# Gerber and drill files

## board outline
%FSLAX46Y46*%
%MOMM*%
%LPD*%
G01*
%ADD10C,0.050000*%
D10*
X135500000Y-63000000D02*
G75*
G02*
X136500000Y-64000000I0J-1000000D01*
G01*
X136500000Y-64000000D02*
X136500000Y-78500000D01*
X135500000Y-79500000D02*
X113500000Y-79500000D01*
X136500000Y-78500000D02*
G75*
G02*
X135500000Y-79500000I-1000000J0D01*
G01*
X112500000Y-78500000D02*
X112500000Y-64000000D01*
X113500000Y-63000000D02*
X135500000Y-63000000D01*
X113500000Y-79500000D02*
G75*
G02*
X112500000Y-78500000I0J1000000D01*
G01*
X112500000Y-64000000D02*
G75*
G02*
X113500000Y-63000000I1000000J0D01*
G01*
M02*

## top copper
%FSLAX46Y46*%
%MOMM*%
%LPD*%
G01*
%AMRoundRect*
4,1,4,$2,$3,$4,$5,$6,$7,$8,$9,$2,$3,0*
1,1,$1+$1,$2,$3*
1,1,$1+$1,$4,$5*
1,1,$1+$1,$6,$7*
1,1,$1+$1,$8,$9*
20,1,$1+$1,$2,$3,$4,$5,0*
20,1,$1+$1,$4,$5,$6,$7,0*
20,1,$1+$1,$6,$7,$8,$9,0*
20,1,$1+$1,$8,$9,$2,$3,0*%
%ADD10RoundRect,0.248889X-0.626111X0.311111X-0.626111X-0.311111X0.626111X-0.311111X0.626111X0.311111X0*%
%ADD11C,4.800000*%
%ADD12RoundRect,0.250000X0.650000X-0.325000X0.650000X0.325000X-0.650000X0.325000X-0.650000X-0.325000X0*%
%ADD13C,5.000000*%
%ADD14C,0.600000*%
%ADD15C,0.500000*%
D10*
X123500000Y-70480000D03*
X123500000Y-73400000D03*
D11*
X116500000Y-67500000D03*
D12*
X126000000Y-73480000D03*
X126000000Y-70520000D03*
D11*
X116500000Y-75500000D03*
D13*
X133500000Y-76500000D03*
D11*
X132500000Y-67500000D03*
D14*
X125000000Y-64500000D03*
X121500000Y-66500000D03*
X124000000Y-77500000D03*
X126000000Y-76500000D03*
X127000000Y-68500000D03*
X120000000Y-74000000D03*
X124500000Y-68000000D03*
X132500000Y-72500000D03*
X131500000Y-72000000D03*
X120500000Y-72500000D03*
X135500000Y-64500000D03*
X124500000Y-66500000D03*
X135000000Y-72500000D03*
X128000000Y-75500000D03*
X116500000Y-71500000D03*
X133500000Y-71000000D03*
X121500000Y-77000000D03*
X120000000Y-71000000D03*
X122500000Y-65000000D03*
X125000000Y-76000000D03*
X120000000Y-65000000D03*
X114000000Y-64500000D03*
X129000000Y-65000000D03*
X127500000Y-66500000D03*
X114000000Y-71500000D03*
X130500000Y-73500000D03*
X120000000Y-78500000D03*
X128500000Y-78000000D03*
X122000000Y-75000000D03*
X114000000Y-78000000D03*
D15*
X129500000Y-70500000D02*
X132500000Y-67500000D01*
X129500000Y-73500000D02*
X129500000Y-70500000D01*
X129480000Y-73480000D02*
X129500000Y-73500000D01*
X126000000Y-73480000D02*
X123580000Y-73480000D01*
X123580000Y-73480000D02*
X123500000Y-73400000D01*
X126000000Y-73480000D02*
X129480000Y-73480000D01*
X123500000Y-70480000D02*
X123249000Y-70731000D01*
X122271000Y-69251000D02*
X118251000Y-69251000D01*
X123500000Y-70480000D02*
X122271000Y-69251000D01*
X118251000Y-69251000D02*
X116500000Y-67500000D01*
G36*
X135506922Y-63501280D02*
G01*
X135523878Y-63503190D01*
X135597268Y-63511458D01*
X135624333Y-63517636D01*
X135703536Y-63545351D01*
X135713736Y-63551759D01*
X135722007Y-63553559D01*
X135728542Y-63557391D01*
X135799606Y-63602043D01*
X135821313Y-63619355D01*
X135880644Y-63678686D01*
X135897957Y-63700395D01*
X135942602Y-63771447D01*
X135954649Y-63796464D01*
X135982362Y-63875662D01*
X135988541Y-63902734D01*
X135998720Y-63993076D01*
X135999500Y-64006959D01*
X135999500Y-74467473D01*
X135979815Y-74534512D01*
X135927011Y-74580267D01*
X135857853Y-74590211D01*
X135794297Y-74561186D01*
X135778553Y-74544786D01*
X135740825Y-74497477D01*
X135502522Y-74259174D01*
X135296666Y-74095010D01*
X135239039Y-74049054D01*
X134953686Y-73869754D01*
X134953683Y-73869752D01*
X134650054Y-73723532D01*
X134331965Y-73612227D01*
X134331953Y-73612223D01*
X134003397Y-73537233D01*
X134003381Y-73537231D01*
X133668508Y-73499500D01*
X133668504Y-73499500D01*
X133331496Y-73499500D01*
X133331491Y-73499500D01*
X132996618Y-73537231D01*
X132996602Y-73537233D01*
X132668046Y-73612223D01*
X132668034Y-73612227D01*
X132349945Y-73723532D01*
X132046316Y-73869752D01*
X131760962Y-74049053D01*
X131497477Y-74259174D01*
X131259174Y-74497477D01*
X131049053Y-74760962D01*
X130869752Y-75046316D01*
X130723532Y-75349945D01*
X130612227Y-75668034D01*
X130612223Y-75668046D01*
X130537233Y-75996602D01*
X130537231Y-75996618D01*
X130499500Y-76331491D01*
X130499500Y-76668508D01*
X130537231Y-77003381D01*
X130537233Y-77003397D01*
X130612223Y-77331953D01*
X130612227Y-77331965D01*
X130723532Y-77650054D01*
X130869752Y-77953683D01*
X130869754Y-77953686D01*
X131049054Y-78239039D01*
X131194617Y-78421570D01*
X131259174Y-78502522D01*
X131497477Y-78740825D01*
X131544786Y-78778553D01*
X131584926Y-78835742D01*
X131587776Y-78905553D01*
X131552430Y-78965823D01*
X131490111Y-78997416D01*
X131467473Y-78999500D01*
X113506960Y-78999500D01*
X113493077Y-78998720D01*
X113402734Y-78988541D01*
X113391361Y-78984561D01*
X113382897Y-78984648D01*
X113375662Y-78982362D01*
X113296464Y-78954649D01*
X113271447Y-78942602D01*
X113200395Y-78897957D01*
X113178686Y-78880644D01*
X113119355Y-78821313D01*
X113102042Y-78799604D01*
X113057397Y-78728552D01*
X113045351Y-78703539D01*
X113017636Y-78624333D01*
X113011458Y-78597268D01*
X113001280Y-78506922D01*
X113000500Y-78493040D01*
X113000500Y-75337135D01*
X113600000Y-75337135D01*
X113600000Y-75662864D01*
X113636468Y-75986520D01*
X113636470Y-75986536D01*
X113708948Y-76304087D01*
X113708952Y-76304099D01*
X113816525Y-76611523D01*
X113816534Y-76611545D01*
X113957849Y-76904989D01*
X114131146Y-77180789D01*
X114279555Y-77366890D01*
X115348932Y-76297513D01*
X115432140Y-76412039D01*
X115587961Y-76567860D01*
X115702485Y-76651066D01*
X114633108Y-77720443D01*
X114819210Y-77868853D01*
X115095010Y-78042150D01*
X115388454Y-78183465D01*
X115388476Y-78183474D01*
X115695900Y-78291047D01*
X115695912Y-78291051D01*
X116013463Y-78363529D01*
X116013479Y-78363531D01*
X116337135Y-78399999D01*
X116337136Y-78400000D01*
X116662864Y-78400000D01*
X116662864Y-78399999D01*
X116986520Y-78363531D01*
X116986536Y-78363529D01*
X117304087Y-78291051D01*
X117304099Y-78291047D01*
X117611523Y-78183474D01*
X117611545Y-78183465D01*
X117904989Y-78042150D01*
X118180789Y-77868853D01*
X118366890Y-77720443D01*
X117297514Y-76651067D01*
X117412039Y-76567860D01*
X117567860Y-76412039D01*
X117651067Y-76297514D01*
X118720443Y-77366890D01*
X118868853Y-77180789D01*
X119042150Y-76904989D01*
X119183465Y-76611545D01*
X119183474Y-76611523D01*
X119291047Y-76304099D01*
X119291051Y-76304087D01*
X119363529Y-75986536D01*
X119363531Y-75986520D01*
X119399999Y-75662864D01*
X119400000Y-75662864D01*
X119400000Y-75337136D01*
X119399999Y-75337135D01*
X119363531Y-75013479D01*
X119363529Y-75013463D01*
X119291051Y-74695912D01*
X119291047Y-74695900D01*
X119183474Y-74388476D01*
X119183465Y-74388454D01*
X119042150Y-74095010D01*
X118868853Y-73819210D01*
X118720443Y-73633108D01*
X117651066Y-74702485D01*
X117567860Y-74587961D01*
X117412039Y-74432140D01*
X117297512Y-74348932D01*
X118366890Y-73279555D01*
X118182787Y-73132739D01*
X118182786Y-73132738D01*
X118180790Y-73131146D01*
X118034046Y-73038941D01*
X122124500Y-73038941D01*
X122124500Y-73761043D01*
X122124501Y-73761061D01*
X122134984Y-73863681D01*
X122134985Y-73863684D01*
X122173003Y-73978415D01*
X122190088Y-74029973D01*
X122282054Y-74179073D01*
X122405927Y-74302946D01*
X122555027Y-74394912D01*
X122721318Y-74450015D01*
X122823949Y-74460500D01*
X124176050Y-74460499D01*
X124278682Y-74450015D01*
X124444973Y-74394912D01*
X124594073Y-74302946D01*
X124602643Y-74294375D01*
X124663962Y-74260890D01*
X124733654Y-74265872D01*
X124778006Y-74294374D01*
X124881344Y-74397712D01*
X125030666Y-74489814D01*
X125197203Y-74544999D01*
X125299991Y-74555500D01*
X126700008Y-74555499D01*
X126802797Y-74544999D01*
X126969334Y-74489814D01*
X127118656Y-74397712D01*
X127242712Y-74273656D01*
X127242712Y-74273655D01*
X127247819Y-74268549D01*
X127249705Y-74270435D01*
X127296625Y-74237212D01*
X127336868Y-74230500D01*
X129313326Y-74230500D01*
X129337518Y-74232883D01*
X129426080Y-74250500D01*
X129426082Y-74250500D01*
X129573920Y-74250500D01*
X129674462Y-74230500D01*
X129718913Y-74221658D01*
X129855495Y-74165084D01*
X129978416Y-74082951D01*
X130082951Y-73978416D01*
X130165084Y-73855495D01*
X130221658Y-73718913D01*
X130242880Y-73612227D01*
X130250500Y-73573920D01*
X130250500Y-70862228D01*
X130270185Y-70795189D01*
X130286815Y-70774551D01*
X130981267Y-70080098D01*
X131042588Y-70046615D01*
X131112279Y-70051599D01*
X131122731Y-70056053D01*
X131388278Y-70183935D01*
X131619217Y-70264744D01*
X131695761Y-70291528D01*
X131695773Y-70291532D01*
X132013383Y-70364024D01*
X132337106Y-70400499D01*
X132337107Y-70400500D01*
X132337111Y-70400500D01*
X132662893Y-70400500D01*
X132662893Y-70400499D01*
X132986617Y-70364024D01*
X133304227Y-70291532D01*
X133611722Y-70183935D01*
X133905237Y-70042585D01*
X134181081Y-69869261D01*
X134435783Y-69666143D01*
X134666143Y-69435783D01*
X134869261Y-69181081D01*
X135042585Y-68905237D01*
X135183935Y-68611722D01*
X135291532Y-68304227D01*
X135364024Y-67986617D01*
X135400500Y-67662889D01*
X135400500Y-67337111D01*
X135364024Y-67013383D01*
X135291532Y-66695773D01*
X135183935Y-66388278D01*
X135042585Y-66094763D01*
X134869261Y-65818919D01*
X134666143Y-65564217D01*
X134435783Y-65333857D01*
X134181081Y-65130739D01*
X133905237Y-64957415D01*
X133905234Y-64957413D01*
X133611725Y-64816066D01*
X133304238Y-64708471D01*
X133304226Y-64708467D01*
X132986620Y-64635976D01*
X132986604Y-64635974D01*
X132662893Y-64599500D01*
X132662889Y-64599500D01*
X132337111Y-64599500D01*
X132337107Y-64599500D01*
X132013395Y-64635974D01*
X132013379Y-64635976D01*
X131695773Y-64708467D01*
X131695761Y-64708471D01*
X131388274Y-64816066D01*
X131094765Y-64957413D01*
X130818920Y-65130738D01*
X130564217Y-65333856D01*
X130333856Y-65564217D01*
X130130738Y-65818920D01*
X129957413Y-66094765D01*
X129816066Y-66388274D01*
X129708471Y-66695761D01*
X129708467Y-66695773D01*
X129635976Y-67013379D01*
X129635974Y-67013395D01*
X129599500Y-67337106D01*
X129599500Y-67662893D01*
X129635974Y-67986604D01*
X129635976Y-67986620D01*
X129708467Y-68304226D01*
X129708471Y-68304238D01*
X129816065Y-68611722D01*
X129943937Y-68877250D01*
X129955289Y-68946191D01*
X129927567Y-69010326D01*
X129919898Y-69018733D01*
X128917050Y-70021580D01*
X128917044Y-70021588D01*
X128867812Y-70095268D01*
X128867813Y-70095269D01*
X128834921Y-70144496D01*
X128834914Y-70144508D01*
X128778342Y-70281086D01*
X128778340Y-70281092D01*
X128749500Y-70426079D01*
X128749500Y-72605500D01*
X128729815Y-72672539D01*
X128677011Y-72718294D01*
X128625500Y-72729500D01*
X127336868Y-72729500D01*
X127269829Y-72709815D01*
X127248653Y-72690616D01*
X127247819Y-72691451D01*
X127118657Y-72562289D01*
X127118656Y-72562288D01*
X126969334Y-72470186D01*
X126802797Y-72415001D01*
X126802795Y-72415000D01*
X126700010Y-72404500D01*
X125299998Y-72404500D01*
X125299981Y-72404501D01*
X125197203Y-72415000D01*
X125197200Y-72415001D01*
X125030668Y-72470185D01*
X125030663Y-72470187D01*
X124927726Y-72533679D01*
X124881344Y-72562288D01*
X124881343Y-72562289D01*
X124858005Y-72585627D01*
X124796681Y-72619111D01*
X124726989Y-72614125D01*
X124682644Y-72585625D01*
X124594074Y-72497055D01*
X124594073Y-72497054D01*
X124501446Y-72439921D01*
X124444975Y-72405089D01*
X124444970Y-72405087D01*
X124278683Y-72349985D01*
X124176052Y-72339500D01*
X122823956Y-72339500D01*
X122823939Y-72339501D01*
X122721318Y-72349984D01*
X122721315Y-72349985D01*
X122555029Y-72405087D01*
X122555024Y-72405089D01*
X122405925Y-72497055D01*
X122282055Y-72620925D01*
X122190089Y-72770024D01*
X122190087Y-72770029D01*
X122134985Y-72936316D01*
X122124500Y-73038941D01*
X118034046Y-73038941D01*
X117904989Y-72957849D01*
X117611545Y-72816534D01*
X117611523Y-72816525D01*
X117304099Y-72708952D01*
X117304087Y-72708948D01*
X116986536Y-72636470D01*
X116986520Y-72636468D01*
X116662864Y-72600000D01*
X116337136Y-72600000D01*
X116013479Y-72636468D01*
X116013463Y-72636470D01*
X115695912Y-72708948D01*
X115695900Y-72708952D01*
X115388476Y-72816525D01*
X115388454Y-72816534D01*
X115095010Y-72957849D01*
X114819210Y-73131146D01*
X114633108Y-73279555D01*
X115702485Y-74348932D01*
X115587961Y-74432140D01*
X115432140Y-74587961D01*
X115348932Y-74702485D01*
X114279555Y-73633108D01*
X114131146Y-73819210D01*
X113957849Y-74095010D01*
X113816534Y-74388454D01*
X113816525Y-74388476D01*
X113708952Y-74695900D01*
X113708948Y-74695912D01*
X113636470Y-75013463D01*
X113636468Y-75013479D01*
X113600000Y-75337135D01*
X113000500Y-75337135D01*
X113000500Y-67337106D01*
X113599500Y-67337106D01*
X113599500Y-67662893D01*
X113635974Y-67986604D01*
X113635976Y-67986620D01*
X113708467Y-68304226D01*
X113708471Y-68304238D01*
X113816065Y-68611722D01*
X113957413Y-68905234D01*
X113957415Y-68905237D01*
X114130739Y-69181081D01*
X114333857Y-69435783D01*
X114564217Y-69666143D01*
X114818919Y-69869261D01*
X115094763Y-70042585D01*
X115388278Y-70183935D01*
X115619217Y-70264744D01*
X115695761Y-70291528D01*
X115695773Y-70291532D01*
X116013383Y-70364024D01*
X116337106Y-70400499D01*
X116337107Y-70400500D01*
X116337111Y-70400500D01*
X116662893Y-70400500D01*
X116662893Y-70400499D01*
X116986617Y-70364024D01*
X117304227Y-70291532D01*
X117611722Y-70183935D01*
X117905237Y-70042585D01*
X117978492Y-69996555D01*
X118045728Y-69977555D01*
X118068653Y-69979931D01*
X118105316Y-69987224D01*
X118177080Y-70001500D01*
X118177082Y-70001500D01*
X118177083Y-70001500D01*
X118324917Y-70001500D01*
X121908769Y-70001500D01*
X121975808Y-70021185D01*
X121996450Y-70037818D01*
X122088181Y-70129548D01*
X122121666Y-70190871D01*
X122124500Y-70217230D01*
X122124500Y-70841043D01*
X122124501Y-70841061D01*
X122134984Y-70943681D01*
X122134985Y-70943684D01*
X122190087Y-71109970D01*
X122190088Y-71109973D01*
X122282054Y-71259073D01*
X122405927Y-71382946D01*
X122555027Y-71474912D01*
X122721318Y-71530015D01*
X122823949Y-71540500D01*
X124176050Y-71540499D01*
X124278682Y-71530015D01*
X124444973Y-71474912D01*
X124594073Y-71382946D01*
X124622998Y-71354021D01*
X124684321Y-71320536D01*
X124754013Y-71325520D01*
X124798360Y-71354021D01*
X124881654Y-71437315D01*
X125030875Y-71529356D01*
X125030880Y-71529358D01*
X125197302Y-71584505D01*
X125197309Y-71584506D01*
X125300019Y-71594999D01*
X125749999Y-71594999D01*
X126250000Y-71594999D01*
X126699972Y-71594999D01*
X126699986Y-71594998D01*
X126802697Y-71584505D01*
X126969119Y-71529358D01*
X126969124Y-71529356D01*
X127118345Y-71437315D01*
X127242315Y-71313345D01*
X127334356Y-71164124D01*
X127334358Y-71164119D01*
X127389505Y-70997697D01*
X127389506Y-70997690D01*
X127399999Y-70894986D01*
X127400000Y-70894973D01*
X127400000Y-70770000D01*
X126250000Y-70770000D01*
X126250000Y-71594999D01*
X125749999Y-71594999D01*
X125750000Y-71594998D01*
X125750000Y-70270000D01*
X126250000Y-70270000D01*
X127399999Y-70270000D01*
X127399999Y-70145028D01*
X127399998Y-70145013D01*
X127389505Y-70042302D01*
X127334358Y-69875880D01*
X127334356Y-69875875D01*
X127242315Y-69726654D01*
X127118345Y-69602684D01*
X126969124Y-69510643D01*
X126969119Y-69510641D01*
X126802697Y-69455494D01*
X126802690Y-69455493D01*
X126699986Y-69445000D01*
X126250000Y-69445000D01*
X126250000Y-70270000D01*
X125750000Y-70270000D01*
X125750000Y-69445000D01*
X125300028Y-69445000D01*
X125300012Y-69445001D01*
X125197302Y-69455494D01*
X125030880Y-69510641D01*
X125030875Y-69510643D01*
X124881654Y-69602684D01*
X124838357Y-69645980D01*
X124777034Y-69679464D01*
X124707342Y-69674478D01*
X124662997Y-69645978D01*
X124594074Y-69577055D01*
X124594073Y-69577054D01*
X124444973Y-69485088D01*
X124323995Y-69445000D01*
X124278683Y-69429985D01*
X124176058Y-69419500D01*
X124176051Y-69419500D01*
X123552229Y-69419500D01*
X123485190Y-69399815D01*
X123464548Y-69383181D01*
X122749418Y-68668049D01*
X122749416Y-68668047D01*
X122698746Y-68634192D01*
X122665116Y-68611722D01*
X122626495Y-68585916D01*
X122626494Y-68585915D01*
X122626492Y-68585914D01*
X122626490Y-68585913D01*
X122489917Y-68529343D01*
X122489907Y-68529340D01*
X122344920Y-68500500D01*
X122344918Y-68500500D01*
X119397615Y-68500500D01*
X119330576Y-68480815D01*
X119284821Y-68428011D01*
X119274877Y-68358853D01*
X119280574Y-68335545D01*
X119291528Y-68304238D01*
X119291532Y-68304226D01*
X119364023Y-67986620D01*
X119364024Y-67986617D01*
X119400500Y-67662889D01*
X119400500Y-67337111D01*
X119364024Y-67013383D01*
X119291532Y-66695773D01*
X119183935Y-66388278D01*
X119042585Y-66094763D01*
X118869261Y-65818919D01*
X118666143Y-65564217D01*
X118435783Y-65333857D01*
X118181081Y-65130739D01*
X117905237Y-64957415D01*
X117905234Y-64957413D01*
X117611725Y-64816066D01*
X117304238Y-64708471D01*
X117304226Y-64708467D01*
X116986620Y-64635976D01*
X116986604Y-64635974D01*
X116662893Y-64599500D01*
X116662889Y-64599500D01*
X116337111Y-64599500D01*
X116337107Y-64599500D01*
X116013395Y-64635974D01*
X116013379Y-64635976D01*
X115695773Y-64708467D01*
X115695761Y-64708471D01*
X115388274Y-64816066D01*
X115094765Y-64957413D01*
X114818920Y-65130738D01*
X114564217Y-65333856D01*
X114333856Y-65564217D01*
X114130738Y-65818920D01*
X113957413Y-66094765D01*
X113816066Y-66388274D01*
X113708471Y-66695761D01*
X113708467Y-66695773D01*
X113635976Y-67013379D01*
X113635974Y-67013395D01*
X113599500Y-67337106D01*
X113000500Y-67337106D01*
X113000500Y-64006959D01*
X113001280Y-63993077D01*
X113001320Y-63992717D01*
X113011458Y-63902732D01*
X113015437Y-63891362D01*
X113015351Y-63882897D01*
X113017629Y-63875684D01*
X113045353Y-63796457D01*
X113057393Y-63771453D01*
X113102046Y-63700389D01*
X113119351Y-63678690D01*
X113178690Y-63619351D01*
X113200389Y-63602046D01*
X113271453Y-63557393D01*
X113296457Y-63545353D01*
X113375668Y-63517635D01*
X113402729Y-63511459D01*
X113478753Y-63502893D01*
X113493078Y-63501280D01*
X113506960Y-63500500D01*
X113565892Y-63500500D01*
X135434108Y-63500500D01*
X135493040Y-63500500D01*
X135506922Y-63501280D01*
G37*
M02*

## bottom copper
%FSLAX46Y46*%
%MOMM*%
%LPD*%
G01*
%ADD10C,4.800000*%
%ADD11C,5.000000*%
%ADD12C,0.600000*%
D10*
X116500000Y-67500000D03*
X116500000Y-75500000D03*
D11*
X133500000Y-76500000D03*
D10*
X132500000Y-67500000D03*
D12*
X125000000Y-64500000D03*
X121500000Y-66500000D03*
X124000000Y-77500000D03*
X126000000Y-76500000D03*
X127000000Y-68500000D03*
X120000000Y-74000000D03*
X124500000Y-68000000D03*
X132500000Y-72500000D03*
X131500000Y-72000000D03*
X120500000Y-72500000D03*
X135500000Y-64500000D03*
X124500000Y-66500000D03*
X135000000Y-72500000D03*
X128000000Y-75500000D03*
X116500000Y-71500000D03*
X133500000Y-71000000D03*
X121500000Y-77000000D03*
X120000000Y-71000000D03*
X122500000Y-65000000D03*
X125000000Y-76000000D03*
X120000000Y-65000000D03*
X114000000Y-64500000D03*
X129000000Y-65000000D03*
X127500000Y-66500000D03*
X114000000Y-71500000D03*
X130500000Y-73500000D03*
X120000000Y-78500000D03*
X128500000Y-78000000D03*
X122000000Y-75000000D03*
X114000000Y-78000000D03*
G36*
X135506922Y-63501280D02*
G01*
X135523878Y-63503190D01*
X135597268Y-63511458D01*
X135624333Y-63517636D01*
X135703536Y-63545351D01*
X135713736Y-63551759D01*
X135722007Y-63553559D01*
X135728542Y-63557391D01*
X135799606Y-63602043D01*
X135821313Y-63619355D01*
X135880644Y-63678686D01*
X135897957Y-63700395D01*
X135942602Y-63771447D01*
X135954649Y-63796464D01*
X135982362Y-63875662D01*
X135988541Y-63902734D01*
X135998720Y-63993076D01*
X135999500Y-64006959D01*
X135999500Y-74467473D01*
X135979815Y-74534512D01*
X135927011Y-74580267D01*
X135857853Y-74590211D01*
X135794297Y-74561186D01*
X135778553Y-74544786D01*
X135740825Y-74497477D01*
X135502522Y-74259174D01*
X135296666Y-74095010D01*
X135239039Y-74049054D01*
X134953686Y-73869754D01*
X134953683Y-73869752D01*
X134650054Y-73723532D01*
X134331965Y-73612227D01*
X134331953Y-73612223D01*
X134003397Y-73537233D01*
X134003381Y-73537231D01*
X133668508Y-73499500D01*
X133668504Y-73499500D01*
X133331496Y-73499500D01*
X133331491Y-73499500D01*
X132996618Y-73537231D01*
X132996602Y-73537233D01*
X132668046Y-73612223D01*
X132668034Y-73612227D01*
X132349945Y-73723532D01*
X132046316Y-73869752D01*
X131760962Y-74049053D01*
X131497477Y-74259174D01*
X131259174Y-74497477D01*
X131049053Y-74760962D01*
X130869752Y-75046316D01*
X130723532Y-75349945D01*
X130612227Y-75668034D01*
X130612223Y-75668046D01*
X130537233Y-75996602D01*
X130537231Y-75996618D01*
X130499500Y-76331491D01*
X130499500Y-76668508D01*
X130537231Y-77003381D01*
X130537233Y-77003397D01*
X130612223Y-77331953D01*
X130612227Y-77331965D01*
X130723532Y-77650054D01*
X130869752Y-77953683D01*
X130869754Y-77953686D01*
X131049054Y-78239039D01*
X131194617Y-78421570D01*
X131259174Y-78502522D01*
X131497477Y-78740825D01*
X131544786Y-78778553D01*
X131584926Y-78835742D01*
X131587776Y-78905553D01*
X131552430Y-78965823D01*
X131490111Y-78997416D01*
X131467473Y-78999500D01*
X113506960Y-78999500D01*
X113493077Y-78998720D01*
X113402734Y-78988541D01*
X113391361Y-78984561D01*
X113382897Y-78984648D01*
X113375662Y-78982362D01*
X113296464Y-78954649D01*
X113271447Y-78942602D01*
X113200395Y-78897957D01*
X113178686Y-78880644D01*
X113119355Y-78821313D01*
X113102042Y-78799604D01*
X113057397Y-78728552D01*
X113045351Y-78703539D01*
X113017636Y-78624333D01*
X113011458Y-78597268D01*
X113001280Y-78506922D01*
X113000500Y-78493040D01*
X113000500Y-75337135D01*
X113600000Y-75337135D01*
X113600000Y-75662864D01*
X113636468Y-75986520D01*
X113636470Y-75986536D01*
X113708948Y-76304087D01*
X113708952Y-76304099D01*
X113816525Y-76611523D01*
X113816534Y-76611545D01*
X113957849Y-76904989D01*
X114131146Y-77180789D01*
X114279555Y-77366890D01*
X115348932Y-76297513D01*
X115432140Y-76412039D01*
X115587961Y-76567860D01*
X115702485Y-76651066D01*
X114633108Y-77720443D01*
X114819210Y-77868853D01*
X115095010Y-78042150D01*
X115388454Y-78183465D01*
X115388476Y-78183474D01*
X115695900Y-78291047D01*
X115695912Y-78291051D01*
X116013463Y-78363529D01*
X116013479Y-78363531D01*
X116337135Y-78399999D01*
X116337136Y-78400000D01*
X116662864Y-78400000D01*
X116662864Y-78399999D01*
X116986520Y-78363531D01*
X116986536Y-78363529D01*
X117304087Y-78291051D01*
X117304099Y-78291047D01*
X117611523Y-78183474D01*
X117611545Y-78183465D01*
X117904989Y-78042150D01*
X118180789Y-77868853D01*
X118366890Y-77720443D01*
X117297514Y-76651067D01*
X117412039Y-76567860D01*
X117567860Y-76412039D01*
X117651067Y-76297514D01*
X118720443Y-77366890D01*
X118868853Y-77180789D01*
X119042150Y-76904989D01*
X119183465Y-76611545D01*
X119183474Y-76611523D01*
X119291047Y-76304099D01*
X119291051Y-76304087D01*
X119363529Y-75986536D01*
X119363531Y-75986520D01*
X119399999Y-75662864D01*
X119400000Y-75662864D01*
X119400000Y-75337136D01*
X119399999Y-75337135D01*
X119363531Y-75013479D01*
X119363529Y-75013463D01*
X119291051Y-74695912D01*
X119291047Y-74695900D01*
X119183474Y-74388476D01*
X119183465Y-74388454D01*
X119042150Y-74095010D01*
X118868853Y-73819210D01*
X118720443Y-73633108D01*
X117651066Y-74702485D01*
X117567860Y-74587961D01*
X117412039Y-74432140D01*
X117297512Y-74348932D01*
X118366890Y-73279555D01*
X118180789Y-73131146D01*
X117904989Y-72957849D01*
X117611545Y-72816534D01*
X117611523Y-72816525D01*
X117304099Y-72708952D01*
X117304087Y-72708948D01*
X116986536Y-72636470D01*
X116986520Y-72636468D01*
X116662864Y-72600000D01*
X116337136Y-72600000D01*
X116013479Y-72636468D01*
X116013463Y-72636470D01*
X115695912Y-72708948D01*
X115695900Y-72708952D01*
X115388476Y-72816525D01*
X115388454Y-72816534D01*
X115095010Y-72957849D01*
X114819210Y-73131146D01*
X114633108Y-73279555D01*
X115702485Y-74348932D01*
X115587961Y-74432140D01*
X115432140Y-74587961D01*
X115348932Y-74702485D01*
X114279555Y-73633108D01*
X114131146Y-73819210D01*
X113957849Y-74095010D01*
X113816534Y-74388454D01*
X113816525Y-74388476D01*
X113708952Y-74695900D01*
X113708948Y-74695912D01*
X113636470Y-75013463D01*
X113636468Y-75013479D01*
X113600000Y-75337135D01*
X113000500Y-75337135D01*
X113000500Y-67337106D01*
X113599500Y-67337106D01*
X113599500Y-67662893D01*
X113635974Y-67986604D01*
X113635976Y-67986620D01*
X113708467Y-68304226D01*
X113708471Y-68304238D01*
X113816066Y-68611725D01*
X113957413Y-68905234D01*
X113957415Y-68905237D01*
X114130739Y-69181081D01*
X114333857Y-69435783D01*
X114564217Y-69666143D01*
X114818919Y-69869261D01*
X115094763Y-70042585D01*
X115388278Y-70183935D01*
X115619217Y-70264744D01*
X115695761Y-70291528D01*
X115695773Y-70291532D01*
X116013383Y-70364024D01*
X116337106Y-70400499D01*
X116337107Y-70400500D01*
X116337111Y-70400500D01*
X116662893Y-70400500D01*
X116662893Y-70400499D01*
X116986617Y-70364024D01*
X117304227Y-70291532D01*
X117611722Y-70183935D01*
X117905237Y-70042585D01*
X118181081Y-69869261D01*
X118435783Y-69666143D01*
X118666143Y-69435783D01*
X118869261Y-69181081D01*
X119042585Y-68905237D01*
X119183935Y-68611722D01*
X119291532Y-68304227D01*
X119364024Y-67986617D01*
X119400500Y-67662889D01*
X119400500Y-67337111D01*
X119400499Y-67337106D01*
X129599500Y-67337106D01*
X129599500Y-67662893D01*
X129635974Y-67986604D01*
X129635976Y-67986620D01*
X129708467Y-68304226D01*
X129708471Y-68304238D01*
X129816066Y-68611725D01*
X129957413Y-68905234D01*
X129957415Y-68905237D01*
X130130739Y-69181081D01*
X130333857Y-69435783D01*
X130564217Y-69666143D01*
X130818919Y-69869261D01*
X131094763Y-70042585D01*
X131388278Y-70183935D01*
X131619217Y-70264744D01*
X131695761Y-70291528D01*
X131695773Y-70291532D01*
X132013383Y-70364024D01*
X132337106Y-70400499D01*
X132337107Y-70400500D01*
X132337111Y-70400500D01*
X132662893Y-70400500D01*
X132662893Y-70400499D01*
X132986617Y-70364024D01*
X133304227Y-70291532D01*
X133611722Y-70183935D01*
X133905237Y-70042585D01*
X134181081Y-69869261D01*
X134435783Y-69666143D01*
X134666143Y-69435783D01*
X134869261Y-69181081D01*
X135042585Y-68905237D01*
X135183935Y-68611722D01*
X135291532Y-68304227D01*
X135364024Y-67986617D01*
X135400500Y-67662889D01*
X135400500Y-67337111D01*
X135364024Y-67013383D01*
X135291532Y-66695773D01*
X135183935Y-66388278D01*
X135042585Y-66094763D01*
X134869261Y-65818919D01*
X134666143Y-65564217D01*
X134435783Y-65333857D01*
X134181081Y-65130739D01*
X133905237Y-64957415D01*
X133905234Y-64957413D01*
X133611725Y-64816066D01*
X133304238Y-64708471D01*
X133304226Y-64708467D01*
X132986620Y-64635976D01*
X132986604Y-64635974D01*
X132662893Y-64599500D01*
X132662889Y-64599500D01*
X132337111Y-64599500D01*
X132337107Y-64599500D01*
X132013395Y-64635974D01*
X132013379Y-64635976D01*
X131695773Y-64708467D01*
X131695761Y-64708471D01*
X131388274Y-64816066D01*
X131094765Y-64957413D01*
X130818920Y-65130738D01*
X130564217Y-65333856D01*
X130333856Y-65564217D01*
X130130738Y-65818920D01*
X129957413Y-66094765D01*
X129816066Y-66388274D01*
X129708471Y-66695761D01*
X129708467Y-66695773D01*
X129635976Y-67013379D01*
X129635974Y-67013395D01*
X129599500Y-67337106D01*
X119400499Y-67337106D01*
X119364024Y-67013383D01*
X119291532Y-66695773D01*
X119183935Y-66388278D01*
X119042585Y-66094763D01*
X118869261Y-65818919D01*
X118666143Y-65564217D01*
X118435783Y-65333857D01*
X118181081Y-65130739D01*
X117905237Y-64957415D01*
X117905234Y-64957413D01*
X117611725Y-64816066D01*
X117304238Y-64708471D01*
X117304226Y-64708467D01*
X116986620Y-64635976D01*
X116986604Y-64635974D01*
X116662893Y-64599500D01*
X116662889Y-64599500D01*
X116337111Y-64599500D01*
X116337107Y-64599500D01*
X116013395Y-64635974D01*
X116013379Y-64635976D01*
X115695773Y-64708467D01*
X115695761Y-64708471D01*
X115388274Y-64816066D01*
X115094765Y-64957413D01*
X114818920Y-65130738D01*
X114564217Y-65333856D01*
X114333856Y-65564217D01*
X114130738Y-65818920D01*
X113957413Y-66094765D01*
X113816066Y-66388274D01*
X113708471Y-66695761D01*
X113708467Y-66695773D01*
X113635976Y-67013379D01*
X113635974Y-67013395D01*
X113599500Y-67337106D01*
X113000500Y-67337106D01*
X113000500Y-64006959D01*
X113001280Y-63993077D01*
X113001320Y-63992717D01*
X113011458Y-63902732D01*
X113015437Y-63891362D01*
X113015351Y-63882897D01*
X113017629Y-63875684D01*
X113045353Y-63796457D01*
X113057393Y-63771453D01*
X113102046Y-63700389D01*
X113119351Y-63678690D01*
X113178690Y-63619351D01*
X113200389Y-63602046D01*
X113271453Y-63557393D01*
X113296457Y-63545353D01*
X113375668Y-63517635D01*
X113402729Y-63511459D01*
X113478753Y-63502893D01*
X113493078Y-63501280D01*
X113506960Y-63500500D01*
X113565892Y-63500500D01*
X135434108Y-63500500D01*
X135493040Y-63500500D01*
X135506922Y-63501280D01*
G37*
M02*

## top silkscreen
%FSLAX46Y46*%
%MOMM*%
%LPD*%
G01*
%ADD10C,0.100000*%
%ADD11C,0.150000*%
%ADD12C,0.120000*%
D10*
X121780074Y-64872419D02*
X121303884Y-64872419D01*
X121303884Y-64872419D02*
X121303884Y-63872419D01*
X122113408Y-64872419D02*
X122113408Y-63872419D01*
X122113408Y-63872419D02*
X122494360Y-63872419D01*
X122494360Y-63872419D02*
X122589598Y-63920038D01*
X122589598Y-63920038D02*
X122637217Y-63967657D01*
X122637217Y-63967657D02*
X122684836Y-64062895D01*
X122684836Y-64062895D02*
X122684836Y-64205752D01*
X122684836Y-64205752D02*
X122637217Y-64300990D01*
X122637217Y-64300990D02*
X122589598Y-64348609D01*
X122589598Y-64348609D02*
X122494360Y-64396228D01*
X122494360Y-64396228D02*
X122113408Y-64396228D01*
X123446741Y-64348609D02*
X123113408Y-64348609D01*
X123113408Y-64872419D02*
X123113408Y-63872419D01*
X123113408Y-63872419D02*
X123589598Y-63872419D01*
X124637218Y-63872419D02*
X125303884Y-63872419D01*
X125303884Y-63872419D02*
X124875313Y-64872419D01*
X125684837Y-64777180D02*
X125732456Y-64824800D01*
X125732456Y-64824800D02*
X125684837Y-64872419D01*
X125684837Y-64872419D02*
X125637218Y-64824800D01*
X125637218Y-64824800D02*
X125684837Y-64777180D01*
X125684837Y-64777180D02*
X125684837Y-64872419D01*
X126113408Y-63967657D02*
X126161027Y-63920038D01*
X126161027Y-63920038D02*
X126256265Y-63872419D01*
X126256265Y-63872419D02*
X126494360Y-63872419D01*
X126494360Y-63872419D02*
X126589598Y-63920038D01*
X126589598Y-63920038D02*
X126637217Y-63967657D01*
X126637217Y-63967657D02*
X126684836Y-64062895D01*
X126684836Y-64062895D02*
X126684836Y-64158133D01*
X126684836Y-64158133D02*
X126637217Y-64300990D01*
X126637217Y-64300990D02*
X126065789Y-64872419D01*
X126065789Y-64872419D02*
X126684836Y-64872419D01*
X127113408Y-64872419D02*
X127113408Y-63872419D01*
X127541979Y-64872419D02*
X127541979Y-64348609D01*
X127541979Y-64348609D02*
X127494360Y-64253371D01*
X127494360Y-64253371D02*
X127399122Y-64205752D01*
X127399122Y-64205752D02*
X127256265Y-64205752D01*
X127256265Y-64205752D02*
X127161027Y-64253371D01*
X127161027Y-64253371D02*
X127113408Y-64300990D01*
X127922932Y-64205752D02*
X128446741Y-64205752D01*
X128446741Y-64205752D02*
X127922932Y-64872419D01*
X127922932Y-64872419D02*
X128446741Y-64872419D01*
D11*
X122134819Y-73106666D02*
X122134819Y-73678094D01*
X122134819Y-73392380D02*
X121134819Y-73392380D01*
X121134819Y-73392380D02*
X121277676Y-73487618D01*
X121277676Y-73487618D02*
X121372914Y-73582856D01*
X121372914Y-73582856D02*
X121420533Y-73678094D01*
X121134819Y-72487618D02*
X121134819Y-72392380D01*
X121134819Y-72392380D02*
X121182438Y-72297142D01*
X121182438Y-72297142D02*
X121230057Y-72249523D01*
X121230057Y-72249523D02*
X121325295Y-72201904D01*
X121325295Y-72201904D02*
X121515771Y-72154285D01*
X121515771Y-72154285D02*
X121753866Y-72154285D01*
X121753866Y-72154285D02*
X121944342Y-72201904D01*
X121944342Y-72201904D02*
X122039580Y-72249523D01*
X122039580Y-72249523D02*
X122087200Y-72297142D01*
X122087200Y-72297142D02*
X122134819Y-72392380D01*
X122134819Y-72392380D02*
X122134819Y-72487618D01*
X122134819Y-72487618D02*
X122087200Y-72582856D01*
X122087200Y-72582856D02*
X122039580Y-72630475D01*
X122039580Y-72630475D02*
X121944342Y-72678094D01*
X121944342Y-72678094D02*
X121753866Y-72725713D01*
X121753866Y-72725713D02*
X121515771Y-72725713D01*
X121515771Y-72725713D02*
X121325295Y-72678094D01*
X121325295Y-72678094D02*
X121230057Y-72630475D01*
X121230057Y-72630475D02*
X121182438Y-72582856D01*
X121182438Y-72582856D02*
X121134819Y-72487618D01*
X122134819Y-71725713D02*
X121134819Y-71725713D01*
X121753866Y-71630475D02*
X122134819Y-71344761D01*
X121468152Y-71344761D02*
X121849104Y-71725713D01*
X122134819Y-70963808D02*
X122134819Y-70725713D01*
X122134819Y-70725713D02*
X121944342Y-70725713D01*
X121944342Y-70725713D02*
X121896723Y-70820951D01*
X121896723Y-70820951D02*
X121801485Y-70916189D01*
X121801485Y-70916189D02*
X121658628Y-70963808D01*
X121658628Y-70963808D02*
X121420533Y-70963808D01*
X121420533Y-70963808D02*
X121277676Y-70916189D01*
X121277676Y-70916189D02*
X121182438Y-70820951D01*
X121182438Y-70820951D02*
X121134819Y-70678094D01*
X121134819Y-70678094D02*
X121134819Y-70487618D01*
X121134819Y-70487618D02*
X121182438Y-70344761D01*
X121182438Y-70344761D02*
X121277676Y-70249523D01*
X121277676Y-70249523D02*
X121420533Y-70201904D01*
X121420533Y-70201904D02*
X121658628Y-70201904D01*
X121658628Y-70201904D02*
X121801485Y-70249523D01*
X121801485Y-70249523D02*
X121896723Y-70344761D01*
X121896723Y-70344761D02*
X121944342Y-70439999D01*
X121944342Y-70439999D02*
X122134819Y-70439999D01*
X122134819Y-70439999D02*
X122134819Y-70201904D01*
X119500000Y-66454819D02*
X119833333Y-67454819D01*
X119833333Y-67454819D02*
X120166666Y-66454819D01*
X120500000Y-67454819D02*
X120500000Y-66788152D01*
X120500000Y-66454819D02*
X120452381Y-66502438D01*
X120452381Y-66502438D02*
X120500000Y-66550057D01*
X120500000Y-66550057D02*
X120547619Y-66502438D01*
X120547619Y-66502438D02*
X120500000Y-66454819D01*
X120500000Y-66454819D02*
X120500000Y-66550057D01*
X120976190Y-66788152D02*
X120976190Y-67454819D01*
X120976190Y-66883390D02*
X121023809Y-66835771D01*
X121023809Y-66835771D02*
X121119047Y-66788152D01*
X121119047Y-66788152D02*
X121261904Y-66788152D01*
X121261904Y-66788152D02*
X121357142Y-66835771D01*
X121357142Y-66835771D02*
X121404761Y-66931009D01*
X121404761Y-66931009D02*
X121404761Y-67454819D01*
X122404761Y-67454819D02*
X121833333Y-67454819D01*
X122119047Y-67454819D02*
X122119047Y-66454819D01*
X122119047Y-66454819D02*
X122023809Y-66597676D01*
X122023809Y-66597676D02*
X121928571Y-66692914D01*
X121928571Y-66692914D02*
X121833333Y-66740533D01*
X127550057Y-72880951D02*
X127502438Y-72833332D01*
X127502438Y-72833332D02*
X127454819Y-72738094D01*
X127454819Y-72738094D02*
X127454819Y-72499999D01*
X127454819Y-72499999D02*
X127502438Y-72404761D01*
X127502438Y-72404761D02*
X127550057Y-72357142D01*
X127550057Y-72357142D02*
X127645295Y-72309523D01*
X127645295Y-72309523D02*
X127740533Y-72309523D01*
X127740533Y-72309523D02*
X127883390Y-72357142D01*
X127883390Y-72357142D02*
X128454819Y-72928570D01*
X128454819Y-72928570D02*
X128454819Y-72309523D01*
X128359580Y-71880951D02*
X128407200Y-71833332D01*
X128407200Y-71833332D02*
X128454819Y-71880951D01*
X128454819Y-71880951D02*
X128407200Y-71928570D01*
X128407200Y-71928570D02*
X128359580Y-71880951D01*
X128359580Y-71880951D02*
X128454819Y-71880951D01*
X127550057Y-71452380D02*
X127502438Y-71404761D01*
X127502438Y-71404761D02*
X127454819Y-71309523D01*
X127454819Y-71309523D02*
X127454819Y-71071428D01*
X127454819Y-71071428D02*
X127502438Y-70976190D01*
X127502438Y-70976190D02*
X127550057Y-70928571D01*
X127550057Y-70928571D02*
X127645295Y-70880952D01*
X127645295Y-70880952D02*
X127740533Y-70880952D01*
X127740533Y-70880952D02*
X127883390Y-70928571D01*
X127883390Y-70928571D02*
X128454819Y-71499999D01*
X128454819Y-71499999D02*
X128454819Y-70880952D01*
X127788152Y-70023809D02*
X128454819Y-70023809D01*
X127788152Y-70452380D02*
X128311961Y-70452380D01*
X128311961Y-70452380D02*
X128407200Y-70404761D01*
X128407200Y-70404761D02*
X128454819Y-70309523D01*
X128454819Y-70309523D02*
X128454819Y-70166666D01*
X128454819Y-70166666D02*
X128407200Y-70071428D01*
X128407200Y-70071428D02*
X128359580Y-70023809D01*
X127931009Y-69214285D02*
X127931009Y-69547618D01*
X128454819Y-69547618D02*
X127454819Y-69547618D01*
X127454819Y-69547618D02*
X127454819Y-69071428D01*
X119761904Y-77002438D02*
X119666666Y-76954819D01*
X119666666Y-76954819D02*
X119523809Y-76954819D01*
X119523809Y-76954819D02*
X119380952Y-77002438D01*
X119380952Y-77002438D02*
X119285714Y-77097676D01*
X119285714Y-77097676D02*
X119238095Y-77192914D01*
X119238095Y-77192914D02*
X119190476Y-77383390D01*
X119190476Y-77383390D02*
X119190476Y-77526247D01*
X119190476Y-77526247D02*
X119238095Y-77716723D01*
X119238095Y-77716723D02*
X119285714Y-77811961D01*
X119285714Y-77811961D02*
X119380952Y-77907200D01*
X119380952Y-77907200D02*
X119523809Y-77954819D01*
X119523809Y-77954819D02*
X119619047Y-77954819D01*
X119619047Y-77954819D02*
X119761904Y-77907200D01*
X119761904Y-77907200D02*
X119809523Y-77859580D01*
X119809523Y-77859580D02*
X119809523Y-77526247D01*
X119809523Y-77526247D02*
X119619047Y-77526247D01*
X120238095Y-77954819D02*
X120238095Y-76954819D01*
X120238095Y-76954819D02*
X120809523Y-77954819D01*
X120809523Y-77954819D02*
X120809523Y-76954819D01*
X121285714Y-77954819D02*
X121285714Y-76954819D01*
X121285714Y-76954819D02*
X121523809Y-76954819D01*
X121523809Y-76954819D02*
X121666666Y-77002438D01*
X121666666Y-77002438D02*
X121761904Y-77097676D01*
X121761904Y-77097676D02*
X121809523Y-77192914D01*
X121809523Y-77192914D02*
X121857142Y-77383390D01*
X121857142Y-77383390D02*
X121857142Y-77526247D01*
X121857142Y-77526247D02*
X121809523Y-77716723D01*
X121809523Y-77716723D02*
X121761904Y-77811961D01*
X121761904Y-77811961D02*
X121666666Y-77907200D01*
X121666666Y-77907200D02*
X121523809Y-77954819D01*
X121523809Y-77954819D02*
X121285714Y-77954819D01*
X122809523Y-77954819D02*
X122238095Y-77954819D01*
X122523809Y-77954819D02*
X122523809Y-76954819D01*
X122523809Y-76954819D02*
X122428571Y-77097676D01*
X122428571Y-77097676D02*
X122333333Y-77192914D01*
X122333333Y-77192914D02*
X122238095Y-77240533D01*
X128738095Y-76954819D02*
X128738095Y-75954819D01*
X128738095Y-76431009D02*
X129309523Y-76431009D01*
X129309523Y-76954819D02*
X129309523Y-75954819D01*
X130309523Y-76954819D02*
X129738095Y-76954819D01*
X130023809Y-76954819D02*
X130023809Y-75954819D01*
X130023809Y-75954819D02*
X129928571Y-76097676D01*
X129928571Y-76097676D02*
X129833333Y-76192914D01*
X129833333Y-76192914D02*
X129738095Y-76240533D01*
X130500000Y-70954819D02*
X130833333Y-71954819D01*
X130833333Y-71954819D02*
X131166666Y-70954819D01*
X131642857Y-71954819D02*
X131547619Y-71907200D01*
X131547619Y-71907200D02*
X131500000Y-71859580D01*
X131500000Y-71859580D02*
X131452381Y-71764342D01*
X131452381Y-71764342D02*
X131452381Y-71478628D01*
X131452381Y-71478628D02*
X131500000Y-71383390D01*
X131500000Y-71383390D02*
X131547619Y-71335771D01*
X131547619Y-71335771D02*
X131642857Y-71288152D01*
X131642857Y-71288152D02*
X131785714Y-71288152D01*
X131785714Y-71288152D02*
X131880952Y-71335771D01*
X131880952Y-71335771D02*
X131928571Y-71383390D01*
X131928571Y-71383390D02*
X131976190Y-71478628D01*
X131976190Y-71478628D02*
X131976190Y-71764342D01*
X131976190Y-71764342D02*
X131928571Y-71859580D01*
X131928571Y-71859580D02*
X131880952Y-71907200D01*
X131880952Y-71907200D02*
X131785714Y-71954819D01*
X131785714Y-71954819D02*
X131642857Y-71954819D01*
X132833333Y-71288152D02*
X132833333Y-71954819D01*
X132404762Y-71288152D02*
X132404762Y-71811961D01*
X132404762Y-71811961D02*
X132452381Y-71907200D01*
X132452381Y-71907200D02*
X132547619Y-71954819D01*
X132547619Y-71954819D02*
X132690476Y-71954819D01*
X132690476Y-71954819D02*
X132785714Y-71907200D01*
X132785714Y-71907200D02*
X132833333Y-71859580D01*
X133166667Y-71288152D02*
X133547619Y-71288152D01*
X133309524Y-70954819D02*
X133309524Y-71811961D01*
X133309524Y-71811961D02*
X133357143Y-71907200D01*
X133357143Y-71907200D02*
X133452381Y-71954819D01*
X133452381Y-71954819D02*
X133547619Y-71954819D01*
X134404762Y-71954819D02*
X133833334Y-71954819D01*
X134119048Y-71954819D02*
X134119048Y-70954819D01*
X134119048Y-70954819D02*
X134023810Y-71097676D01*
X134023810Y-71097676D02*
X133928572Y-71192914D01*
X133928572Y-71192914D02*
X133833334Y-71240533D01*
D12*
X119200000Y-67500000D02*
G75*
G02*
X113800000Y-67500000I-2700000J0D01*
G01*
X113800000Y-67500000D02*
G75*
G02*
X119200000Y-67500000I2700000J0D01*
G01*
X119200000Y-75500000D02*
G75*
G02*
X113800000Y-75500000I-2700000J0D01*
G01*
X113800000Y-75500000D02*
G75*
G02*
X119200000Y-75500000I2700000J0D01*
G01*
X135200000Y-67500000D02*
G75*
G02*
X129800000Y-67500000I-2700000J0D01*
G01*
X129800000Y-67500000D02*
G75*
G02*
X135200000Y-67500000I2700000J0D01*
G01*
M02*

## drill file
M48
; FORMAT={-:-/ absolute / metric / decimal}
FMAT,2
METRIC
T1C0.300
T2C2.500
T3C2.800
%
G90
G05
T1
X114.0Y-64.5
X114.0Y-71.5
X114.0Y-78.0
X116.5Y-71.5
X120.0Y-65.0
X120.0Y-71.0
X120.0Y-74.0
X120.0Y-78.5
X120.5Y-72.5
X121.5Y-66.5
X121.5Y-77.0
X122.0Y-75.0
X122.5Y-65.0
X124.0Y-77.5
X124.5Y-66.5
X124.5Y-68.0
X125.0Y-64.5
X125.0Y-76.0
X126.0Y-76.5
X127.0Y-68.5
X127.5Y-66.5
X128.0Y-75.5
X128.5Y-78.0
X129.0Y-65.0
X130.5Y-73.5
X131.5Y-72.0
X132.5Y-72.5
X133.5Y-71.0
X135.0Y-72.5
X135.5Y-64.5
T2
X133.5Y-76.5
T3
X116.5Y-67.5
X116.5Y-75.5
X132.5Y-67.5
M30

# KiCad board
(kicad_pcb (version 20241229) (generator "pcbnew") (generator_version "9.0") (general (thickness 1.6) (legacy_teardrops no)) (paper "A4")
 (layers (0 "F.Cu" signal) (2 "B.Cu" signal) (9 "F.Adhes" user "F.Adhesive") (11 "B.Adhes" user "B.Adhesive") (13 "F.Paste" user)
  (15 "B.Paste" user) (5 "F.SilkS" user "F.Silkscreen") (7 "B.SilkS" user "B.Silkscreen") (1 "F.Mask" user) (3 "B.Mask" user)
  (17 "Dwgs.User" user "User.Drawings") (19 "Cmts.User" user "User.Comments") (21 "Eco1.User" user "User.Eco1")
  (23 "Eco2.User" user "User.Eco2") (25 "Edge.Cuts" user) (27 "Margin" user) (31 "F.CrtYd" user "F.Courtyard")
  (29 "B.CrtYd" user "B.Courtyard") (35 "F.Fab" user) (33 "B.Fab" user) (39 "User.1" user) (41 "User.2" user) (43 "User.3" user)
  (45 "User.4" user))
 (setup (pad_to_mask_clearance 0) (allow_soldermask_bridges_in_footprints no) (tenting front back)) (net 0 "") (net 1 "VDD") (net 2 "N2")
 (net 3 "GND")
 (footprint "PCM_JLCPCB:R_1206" (layer "F.Cu") (at 123.5 71.94 -90)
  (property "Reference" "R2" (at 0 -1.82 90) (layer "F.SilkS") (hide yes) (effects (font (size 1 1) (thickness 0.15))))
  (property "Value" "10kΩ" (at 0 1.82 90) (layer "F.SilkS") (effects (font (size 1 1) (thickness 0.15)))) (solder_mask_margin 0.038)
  (pad "1" smd roundrect (at -1.46 0 270) (size 1.12 1.75) (layers "F.Cu" "F.Mask" "F.Paste") (roundrect_rratio 0.222222) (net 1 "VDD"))
  (pad "2" smd roundrect (at 1.46 0 270) (size 1.12 1.75) (layers "F.Cu" "F.Mask" "F.Paste") (roundrect_rratio 0.222222) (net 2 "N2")))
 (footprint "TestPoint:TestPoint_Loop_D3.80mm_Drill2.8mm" (layer "F.Cu") (at 116.5 67.5)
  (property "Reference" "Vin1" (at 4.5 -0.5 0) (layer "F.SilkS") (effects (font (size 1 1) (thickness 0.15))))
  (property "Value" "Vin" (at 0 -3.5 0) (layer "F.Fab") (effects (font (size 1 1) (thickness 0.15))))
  (fp_circle (center 0 0) (end 2.7 0) (stroke (width 0.12) (type solid)) (fill no) (layer "F.SilkS"))
  (pad "1" thru_hole circle (at 0 0) (size 4.8 4.8) (drill 2.8) (layers "*.Cu" "*.Mask") (remove_unused_layers no) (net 1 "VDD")))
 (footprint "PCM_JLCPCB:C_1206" (layer "F.Cu") (at 126 72 90)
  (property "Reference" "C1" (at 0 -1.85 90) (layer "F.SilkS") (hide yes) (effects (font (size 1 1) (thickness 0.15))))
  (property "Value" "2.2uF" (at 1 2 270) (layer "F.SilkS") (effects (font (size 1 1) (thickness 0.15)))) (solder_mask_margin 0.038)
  (pad "1" smd roundrect (at -1.48 0 90) (size 1.15 1.8) (layers "F.Cu" "F.Mask" "F.Paste") (roundrect_rratio 0.217391) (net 2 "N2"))
  (pad "2" smd roundrect (at 1.48 0 90) (size 1.15 1.8) (layers "F.Cu" "F.Mask" "F.Paste") (roundrect_rratio 0.217391) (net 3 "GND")))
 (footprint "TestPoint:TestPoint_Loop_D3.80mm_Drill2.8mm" (layer "F.Cu") (at 116.5 75.5)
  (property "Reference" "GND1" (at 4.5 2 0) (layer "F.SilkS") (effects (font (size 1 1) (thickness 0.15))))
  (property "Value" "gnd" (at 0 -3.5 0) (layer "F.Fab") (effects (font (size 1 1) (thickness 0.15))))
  (fp_circle (center 0 0) (end 2.7 0) (stroke (width 0.12) (type solid)) (fill no) (layer "F.SilkS"))
  (pad "1" thru_hole circle (at 0 0) (size 4.8 4.8) (drill 2.8) (layers "*.Cu" "*.Mask") (remove_unused_layers no) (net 3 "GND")))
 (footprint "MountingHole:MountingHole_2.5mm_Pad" (layer "F.Cu") (at 133.5 76.5)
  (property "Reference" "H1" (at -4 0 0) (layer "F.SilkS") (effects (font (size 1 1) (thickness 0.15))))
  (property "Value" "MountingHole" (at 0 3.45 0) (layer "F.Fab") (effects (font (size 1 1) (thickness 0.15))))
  (pad "1" thru_hole circle (at 0 0) (size 5 5) (drill 2.5) (layers "*.Cu" "*.Mask") (remove_unused_layers no) (zone_connect 2)))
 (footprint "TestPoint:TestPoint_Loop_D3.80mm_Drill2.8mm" (layer "F.Cu") (at 132.5 67.5)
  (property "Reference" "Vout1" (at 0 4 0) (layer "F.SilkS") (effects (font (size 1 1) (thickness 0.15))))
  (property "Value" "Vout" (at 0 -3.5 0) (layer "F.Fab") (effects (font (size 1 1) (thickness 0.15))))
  (fp_circle (center 0 0) (end 2.7 0) (stroke (width 0.12) (type solid)) (fill no) (layer "F.SilkS"))
  (pad "1" thru_hole circle (at 0 0) (size 4.8 4.8) (drill 2.8) (layers "*.Cu" "*.Mask") (remove_unused_layers no) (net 2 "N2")))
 (gr_arc (start 135.5 63) (mid 136.207107 63.292893) (end 136.5 64) (stroke (width 0.05) (type default)) (layer "Edge.Cuts"))
 (gr_line (start 136.5 64) (end 136.5 78.5) (stroke (width 0.05) (type default)) (layer "Edge.Cuts"))
 (gr_line (start 135.5 79.5) (end 113.5 79.5) (stroke (width 0.05) (type default)) (layer "Edge.Cuts"))
 (gr_arc (start 136.5 78.5) (mid 136.207107 79.207107) (end 135.5 79.5) (stroke (width 0.05) (type default)) (layer "Edge.Cuts"))
 (gr_line (start 112.5 78.5) (end 112.5 64) (stroke (width 0.05) (type default)) (layer "Edge.Cuts"))
 (gr_line (start 113.5 63) (end 135.5 63) (stroke (width 0.05) (type default)) (layer "Edge.Cuts"))
 (gr_arc (start 113.5 79.5) (mid 112.792893 79.207107) (end 112.5 78.5) (stroke (width 0.05) (type default)) (layer "Edge.Cuts"))
 (gr_arc (start 112.5 64) (mid 112.792893 63.292893) (end 113.5 63) (stroke (width 0.05) (type default)) (layer "Edge.Cuts"))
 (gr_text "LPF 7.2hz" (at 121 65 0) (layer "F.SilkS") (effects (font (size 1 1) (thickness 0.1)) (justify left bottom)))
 (via (at 125 64.5) (size 0.6) (drill 0.3) (layers "F.Cu" "B.Cu") (free yes) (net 3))
 (via (at 121.5 66.5) (size 0.6) (drill 0.3) (layers "F.Cu" "B.Cu") (free yes) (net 3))
 (via (at 124 77.5) (size 0.6) (drill 0.3) (layers "F.Cu" "B.Cu") (free yes) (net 3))
 (via (at 126 76.5) (size 0.6) (drill 0.3) (layers "F.Cu" "B.Cu") (free yes) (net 3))
 (via (at 127 68.5) (size 0.6) (drill 0.3) (layers "F.Cu" "B.Cu") (free yes) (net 3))
 (via (at 120 74) (size 0.6) (drill 0.3) (layers "F.Cu" "B.Cu") (free yes) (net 3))
 (via (at 124.5 68) (size 0.6) (drill 0.3) (layers "F.Cu" "B.Cu") (free yes) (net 3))
 (via (at 132.5 72.5) (size 0.6) (drill 0.3) (layers "F.Cu" "B.Cu") (free yes) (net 3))
 (via (at 131.5 72) (size 0.6) (drill 0.3) (layers "F.Cu" "B.Cu") (free yes) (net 3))
 (via (at 120.5 72.5) (size 0.6) (drill 0.3) (layers "F.Cu" "B.Cu") (free yes) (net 3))
 (via (at 135.5 64.5) (size 0.6) (drill 0.3) (layers "F.Cu" "B.Cu") (free yes) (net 3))
 (via (at 124.5 66.5) (size 0.6) (drill 0.3) (layers "F.Cu" "B.Cu") (free yes) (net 3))
 (via (at 135 72.5) (size 0.6) (drill 0.3) (layers "F.Cu" "B.Cu") (free yes) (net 3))
 (via (at 128 75.5) (size 0.6) (drill 0.3) (layers "F.Cu" "B.Cu") (free yes) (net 3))
 (via (at 116.5 71.5) (size 0.6) (drill 0.3) (layers "F.Cu" "B.Cu") (free yes) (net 3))
 (via (at 133.5 71) (size 0.6) (drill 0.3) (layers "F.Cu" "B.Cu") (free yes) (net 3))
 (via (at 121.5 77) (size 0.6) (drill 0.3) (layers "F.Cu" "B.Cu") (free yes) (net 3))
 (via (at 120 71) (size 0.6) (drill 0.3) (layers "F.Cu" "B.Cu") (free yes) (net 3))
 (via (at 122.5 65) (size 0.6) (drill 0.3) (layers "F.Cu" "B.Cu") (free yes) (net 3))
 (via (at 125 76) (size 0.6) (drill 0.3) (layers "F.Cu" "B.Cu") (free yes) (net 3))
 (via (at 120 65) (size 0.6) (drill 0.3) (layers "F.Cu" "B.Cu") (free yes) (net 3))
 (via (at 114 64.5) (size 0.6) (drill 0.3) (layers "F.Cu" "B.Cu") (free yes) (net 3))
 (via (at 129 65) (size 0.6) (drill 0.3) (layers "F.Cu" "B.Cu") (free yes) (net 3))
 (via (at 127.5 66.5) (size 0.6) (drill 0.3) (layers "F.Cu" "B.Cu") (free yes) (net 3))
 (via (at 114 71.5) (size 0.6) (drill 0.3) (layers "F.Cu" "B.Cu") (free yes) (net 3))
 (via (at 130.5 73.5) (size 0.6) (drill 0.3) (layers "F.Cu" "B.Cu") (free yes) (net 3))
 (via (at 120 78.5) (size 0.6) (drill 0.3) (layers "F.Cu" "B.Cu") (free yes) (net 3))
 (via (at 128.5 78) (size 0.6) (drill 0.3) (layers "F.Cu" "B.Cu") (free yes) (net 3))
 (via (at 122 75) (size 0.6) (drill 0.3) (layers "F.Cu" "B.Cu") (free yes) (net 3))
 (via (at 114 78) (size 0.6) (drill 0.3) (layers "F.Cu" "B.Cu") (free yes) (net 3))
 (segment (start 129.5 70.5) (end 132.5 67.5) (width 0.5) (layer "F.Cu") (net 2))
 (segment (start 129.5 73.5) (end 129.5 70.5) (width 0.5) (layer "F.Cu") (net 2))
 (segment (start 129.48 73.48) (end 129.5 73.5) (width 0.5) (layer "F.Cu") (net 2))
 (segment (start 126 73.48) (end 123.58 73.48) (width 0.5) (layer "F.Cu") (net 2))
 (segment (start 123.58 73.48) (end 123.5 73.4) (width 0.5) (layer "F.Cu") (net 2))
 (segment (start 126 73.48) (end 129.48 73.48) (width 0.5) (layer "F.Cu") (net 2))
 (segment (start 123.5 70.48) (end 123.249 70.731) (width 0.5) (layer "F.Cu") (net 1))
 (segment (start 122.271 69.251) (end 118.251 69.251) (width 0.5) (layer "F.Cu") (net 1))
 (segment (start 123.5 70.48) (end 122.271 69.251) (width 0.5) (layer "F.Cu") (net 1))
 (segment (start 118.251 69.251) (end 116.5 67.5) (width 0.5) (layer "F.Cu") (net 1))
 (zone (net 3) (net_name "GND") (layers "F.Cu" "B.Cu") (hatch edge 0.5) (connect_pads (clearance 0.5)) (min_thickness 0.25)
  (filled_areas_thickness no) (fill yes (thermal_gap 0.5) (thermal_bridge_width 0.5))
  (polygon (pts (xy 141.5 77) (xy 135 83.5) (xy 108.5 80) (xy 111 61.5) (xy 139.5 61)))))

